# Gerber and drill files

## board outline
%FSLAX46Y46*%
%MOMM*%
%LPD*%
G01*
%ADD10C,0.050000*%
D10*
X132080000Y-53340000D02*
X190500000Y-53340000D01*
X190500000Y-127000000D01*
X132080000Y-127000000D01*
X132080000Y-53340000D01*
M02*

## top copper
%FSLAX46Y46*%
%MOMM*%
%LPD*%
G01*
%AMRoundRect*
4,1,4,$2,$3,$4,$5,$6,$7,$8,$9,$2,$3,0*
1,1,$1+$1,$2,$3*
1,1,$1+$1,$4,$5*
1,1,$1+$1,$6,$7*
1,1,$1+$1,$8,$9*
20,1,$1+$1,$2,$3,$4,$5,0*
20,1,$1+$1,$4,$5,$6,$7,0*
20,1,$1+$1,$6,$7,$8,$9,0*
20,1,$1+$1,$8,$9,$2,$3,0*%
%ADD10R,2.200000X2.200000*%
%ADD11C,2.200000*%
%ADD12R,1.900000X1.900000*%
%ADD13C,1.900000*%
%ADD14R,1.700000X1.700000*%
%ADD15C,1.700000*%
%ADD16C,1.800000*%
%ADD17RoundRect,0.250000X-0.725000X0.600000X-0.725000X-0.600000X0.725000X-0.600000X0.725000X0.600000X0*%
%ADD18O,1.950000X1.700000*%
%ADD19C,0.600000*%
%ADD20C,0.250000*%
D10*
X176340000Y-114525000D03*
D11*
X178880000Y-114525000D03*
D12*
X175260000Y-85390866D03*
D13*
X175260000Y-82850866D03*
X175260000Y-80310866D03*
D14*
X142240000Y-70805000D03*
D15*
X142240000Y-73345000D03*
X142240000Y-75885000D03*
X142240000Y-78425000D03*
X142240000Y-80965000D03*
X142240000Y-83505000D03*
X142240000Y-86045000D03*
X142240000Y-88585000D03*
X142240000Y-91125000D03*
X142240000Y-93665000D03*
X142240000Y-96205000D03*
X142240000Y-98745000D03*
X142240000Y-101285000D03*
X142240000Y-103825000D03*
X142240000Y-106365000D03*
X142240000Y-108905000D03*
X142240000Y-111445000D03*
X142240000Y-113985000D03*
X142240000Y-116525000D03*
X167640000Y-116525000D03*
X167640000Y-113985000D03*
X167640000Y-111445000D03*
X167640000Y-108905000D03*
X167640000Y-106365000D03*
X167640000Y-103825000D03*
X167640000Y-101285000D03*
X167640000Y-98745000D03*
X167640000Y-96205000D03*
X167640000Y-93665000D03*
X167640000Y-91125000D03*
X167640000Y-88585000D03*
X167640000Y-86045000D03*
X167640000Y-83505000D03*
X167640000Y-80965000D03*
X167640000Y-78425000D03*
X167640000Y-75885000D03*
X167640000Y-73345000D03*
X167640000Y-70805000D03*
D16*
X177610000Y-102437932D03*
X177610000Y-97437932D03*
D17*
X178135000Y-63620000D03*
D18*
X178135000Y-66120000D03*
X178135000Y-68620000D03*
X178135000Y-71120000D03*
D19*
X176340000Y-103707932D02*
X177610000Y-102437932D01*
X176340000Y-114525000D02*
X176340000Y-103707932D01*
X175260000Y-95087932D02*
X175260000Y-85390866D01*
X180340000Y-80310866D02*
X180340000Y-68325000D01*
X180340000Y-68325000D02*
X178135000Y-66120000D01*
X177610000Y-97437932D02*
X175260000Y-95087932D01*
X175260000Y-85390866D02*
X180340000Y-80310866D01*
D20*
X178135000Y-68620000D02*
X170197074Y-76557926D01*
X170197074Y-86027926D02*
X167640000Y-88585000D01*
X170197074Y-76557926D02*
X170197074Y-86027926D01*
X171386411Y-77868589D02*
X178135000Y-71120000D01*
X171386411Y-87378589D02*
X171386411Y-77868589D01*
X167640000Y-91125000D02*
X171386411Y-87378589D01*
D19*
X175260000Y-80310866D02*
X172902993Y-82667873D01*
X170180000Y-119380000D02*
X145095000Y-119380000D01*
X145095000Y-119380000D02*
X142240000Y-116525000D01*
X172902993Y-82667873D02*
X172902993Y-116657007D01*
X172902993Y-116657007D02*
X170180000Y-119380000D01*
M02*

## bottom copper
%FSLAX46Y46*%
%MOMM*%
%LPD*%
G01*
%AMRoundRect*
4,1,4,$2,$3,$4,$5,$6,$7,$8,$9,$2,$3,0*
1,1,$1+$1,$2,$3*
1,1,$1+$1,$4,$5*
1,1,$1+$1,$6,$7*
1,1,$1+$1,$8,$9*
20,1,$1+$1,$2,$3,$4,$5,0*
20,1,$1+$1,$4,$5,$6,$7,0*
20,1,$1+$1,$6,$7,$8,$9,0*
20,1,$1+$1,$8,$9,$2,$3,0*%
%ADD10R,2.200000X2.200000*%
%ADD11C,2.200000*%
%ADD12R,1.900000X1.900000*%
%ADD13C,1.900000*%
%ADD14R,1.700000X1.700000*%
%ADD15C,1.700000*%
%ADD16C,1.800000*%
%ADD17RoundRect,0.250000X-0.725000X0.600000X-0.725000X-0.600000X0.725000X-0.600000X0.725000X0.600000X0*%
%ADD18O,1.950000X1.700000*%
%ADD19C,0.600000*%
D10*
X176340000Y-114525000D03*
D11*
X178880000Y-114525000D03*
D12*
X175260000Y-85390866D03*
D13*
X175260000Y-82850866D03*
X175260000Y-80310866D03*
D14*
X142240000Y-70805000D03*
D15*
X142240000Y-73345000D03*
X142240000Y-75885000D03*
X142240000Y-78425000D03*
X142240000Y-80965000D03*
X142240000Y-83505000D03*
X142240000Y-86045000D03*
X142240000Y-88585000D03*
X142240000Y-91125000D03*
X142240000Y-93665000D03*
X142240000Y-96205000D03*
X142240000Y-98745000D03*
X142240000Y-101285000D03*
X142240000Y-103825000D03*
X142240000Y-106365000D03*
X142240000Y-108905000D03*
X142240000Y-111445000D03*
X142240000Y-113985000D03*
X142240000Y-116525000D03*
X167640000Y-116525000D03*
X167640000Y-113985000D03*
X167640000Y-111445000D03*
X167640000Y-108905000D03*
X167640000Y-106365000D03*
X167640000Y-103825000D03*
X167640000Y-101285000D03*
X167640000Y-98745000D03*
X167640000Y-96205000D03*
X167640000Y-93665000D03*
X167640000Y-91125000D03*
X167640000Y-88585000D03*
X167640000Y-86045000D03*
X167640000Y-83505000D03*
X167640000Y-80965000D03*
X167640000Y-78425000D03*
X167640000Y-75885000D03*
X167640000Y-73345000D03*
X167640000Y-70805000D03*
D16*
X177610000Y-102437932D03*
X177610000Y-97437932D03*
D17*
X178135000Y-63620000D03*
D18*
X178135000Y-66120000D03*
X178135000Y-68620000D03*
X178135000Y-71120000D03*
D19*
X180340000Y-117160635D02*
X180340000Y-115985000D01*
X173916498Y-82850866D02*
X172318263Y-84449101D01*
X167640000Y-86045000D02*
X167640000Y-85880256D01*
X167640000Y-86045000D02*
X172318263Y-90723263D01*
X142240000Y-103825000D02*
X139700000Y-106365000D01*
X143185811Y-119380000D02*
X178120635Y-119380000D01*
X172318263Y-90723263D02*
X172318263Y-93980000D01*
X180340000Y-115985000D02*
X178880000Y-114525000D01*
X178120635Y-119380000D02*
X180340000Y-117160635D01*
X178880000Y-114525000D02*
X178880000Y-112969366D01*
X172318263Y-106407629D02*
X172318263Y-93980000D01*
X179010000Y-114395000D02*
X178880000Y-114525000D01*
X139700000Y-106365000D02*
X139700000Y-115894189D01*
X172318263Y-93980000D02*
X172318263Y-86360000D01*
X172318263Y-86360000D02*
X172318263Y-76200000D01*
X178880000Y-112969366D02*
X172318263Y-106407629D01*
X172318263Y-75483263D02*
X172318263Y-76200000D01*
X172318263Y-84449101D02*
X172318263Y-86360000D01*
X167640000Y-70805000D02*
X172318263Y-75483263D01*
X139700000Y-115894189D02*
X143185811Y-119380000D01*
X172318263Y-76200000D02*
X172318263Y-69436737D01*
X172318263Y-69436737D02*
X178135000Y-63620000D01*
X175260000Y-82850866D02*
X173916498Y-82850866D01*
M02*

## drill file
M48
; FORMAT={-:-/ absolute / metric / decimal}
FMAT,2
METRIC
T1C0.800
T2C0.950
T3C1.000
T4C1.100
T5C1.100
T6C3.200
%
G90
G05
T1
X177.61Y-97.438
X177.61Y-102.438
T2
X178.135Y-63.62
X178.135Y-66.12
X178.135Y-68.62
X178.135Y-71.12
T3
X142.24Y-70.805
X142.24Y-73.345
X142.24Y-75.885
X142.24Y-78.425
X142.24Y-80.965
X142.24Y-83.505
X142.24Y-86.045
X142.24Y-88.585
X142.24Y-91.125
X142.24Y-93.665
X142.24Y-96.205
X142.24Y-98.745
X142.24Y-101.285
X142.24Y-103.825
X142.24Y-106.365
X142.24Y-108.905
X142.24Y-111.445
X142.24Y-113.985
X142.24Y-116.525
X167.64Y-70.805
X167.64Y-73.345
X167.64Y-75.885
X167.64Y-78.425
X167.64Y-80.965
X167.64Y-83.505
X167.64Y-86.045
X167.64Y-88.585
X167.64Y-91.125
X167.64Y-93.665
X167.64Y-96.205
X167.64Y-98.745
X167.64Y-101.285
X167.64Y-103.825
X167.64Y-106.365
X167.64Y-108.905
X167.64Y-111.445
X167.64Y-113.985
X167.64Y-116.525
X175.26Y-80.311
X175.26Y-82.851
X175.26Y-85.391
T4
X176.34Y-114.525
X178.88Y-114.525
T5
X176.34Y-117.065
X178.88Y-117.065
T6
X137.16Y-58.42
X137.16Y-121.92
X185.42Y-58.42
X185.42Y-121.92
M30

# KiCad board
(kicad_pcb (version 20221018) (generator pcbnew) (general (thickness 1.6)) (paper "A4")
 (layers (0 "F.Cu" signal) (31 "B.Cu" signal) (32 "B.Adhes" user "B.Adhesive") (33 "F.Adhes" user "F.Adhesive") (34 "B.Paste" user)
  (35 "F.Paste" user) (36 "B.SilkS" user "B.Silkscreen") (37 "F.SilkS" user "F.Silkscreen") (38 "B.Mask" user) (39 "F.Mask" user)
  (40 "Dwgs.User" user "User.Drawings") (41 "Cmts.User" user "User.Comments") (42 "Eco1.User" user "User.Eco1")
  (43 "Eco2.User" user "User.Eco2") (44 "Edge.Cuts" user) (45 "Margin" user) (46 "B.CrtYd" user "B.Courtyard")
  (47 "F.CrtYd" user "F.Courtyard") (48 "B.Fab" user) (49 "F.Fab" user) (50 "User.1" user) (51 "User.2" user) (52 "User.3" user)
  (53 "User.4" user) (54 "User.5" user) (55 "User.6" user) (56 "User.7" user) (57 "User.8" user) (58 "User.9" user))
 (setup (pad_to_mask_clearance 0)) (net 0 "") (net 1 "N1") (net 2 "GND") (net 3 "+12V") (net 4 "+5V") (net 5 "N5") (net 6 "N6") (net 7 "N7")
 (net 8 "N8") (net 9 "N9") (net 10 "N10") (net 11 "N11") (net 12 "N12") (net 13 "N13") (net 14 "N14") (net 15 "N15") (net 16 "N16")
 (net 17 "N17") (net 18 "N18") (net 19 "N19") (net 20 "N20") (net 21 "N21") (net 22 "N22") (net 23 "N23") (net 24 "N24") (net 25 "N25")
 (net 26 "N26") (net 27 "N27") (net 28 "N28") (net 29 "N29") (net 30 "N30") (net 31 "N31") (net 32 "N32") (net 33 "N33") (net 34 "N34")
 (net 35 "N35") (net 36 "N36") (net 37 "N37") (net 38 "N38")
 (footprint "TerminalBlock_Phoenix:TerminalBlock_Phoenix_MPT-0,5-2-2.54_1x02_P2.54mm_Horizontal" (layer "F.Cu") (at 176.34 114.525)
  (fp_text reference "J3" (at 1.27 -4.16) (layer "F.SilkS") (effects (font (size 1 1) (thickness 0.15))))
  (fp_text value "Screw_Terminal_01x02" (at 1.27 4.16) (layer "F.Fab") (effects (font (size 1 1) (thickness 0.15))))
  (pad "" np_thru_hole circle (at 0 2.54) (size 1.1 1.1) (drill 1.1) (layers "*.Cu" "*.Mask"))
  (pad "" np_thru_hole circle (at 2.54 2.54) (size 1.1 1.1) (drill 1.1) (layers "*.Cu" "*.Mask"))
  (pad "1" thru_hole rect (at 0 0) (size 2.2 2.2) (drill 1.1) (layers "*.Cu" "*.Mask") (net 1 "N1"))
  (pad "2" thru_hole circle (at 2.54 0) (size 2.2 2.2) (drill 1.1) (layers "*.Cu" "*.Mask") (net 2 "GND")))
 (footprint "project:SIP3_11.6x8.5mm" (layer "F.Cu") (at 175.26 85.390866 90)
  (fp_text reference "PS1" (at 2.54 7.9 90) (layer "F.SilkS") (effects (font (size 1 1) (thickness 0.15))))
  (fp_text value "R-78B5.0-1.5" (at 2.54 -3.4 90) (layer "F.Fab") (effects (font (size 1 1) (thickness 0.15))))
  (pad "1" thru_hole rect (at 0 0) (size 1.9 1.9) (drill 1) (layers "*.Cu" "*.Mask") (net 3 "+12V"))
  (pad "2" thru_hole circle (at 2.54 0 270) (size 1.9 1.9) (drill 1) (layers "*.Cu" "*.Mask") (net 2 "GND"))
  (pad "3" thru_hole circle (at 5.08 0) (size 1.9 1.9) (drill 1) (layers "*.Cu" "*.Mask") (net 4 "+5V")))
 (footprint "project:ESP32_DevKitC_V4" (layer "F.Cu") (at 142.24 70.805)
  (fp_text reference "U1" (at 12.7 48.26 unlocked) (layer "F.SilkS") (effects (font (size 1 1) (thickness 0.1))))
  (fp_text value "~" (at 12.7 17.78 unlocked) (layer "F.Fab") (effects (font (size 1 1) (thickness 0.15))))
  (pad "1" thru_hole rect (at 0 0 270) (size 1.7 1.7) (drill 1) (layers "*.Cu" "*.Mask") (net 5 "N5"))
  (pad "2" thru_hole circle (at 0 2.54 270) (size 1.7 1.7) (drill 1) (layers "*.Cu" "*.Mask") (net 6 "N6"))
  (pad "3" thru_hole circle (at 0 5.08 270) (size 1.7 1.7) (drill 1) (layers "*.Cu" "*.Mask") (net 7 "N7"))
  (pad "4" thru_hole circle (at 0 7.62 270) (size 1.7 1.7) (drill 1) (layers "*.Cu" "*.Mask") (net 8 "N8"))
  (pad "5" thru_hole circle (at 0 10.16 270) (size 1.7 1.7) (drill 1) (layers "*.Cu" "*.Mask") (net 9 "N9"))
  (pad "6" thru_hole circle (at 0 12.7 270) (size 1.7 1.7) (drill 1) (layers "*.Cu" "*.Mask") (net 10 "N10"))
  (pad "7" thru_hole circle (at 0 15.24 270) (size 1.7 1.7) (drill 1) (layers "*.Cu" "*.Mask") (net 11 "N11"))
  (pad "8" thru_hole circle (at 0 17.78 270) (size 1.7 1.7) (drill 1) (layers "*.Cu" "*.Mask") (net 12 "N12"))
  (pad "9" thru_hole circle (at 0 20.32 270) (size 1.7 1.7) (drill 1) (layers "*.Cu" "*.Mask") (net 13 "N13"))
  (pad "10" thru_hole circle (at 0 22.86 270) (size 1.7 1.7) (drill 1) (layers "*.Cu" "*.Mask") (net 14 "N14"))
  (pad "11" thru_hole circle (at 0 25.4 270) (size 1.7 1.7) (drill 1) (layers "*.Cu" "*.Mask") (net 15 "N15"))
  (pad "12" thru_hole circle (at 0 27.94 270) (size 1.7 1.7) (drill 1) (layers "*.Cu" "*.Mask") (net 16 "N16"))
  (pad "13" thru_hole circle (at 0 30.48 270) (size 1.7 1.7) (drill 1) (layers "*.Cu" "*.Mask") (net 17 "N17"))
  (pad "14" thru_hole circle (at 0 33.02 270) (size 1.7 1.7) (drill 1) (layers "*.Cu" "*.Mask") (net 2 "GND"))
  (pad "15" thru_hole circle (at 0 35.56 270) (size 1.7 1.7) (drill 1) (layers "*.Cu" "*.Mask") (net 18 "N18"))
  (pad "16" thru_hole circle (at 0 38.1 270) (size 1.7 1.7) (drill 1) (layers "*.Cu" "*.Mask") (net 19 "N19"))
  (pad "17" thru_hole circle (at 0 40.64 270) (size 1.7 1.7) (drill 1) (layers "*.Cu" "*.Mask") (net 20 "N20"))
  (pad "18" thru_hole circle (at 0 43.18 270) (size 1.7 1.7) (drill 1) (layers "*.Cu" "*.Mask") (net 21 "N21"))
  (pad "19" thru_hole circle (at 0 45.72 270) (size 1.7 1.7) (drill 1) (layers "*.Cu" "*.Mask") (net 4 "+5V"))
  (pad "20" thru_hole circle (at 25.4 45.72 270) (size 1.7 1.7) (drill 1) (layers "*.Cu" "*.Mask") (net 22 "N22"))
  (pad "21" thru_hole circle (at 25.4 43.18 270) (size 1.7 1.7) (drill 1) (layers "*.Cu" "*.Mask") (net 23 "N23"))
  (pad "22" thru_hole circle (at 25.4 40.64 270) (size 1.7 1.7) (drill 1) (layers "*.Cu" "*.Mask") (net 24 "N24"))
  (pad "23" thru_hole circle (at 25.4 38.1 270) (size 1.7 1.7) (drill 1) (layers "*.Cu" "*.Mask") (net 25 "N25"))
  (pad "24" thru_hole circle (at 25.4 35.56 270) (size 1.7 1.7) (drill 1) (layers "*.Cu" "*.Mask") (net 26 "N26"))
  (pad "25" thru_hole circle (at 25.4 33.02 270) (size 1.7 1.7) (drill 1) (layers "*.Cu" "*.Mask") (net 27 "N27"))
  (pad "26" thru_hole circle (at 25.4 30.48 270) (size 1.7 1.7) (drill 1) (layers "*.Cu" "*.Mask") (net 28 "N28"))
  (pad "27" thru_hole circle (at 25.4 27.94 270) (size 1.7 1.7) (drill 1) (layers "*.Cu" "*.Mask") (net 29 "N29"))
  (pad "28" thru_hole circle (at 25.4 25.4 270) (size 1.7 1.7) (drill 1) (layers "*.Cu" "*.Mask") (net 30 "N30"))
  (pad "29" thru_hole circle (at 25.4 22.86 270) (size 1.7 1.7) (drill 1) (layers "*.Cu" "*.Mask") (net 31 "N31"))
  (pad "30" thru_hole circle (at 25.4 20.32 270) (size 1.7 1.7) (drill 1) (layers "*.Cu" "*.Mask") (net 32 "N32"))
  (pad "31" thru_hole circle (at 25.4 17.78 270) (size 1.7 1.7) (drill 1) (layers "*.Cu" "*.Mask") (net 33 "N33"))
  (pad "32" thru_hole circle (at 25.4 15.24 270) (size 1.7 1.7) (drill 1) (layers "*.Cu" "*.Mask") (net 2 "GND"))
  (pad "33" thru_hole circle (at 25.4 12.7 270) (size 1.7 1.7) (drill 1) (layers "*.Cu" "*.Mask") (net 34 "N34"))
  (pad "34" thru_hole circle (at 25.4 10.16 270) (size 1.7 1.7) (drill 1) (layers "*.Cu" "*.Mask") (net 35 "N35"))
  (pad "35" thru_hole circle (at 25.4 7.62 270) (size 1.7 1.7) (drill 1) (layers "*.Cu" "*.Mask") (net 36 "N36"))
  (pad "36" thru_hole circle (at 25.4 5.08 270) (size 1.7 1.7) (drill 1) (layers "*.Cu" "*.Mask") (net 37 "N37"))
  (pad "37" thru_hole circle (at 25.4 2.54 270) (size 1.7 1.7) (drill 1) (layers "*.Cu" "*.Mask") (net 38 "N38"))
  (pad "38" thru_hole circle (at 25.4 0 270) (size 1.7 1.7) (drill 1) (layers "*.Cu" "*.Mask") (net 2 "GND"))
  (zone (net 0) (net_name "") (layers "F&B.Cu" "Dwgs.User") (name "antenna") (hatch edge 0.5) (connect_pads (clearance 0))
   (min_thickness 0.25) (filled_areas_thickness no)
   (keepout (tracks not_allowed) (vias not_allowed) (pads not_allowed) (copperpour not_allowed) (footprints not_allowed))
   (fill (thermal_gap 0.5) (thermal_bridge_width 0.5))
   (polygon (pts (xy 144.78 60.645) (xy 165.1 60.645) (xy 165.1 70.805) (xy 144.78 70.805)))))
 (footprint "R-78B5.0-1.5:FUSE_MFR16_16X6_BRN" (layer "F.Cu") (at 177.61 102.437932 90)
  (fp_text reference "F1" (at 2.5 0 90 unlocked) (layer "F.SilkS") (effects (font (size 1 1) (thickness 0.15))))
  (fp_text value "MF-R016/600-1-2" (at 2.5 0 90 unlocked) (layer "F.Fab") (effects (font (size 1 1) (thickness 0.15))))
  (pad "1" thru_hole circle (at 0 0 90) (size 1.8 1.8) (drill 0.8) (layers "*.Cu" "*.Mask") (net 1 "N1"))
  (pad "2" thru_hole circle (at 5 0 90) (size 1.8 1.8) (drill 0.8) (layers "*.Cu" "*.Mask") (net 3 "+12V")))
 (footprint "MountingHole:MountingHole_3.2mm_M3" (layer "F.Cu") (at 185.42 58.42)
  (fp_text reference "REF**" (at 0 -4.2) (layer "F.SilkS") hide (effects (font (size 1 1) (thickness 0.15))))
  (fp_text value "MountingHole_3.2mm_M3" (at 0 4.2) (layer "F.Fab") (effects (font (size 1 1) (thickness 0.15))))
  (pad "" np_thru_hole circle (at 0 0) (size 3.2 3.2) (drill 3.2) (layers "*.Cu" "*.Mask")))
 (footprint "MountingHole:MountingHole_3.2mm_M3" (layer "F.Cu") (at 137.16 121.92)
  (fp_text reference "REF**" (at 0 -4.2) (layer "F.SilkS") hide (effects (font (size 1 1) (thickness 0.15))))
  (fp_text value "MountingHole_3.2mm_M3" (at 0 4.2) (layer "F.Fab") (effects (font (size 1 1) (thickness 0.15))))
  (pad "" np_thru_hole circle (at 0 0) (size 3.2 3.2) (drill 3.2) (layers "F&B.Cu" "*.Mask")))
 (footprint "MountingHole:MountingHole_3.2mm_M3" (layer "F.Cu") (at 137.16 58.42)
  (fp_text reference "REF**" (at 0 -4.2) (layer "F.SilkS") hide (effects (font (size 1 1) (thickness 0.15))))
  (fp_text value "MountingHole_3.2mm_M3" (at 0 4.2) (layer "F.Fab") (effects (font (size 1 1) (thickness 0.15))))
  (pad "" np_thru_hole circle (at 0 0) (size 3.2 3.2) (drill 3.2) (layers "F&B.Cu" "*.Mask")))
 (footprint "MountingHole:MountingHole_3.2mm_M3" (layer "F.Cu") (at 185.42 121.92)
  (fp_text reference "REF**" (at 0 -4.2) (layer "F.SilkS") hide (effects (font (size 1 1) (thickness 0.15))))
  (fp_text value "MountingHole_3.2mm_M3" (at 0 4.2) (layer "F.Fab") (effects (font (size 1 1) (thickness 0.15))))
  (pad "" np_thru_hole circle (at 0 0) (size 3.2 3.2) (drill 3.2) (layers "F&B.Cu" "*.Mask")))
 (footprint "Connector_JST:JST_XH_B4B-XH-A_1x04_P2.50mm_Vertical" (layer "F.Cu") (at 178.135 63.62 -90)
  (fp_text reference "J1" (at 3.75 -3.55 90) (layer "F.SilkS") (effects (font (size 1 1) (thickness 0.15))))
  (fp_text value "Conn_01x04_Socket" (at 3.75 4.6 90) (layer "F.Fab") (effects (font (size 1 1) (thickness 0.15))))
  (pad "1" thru_hole roundrect (at 0 0 270) (size 1.7 1.95) (drill 0.95) (layers "*.Cu" "*.Mask") (roundrect_rratio 0.1470588235)
   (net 2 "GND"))
  (pad "2" thru_hole oval (at 2.5 0 270) (size 1.7 1.95) (drill 0.95) (layers "*.Cu" "*.Mask") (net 3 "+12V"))
  (pad "3" thru_hole oval (at 5 0 270) (size 1.7 1.95) (drill 0.95) (layers "*.Cu" "*.Mask") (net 33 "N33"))
  (pad "4" thru_hole oval (at 7.5 0 270) (size 1.7 1.95) (drill 0.95) (layers "*.Cu" "*.Mask") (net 32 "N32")))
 (gr_rect (start 132.08 53.34) (end 190.5 127) (stroke (width 0.05) (type default)) (fill none) (layer "Edge.Cuts"))
 (segment (start 176.34 103.707932) (end 177.61 102.437932) (width 0.6) (layer "F.Cu") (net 1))
 (segment (start 176.34 114.525) (end 176.34 103.707932) (width 0.6) (layer "F.Cu") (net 1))
 (segment (start 175.26 95.087932) (end 175.26 85.390866) (width 0.6) (layer "F.Cu") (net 3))
 (segment (start 180.34 80.310866) (end 180.34 68.325) (width 0.6) (layer "F.Cu") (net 3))
 (segment (start 180.34 68.325) (end 178.135 66.12) (width 0.6) (layer "F.Cu") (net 3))
 (segment (start 177.61 97.437932) (end 175.26 95.087932) (width 0.6) (layer "F.Cu") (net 3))
 (segment (start 175.26 85.390866) (end 180.34 80.310866) (width 0.6) (layer "F.Cu") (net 3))
 (segment (start 180.34 117.160635) (end 180.34 115.985) (width 0.6) (layer "B.Cu") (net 2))
 (segment (start 173.916498 82.850866) (end 172.318263 84.449101) (width 0.6) (layer "B.Cu") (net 2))
 (segment (start 167.64 86.045) (end 167.64 85.880256) (width 0.6) (layer "B.Cu") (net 2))
 (segment (start 167.64 86.045) (end 172.318263 90.723263) (width 0.6) (layer "B.Cu") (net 2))
 (segment (start 142.24 103.825) (end 139.7 106.365) (width 0.6) (layer "B.Cu") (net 2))
 (segment (start 143.185811 119.38) (end 178.120635 119.38) (width 0.6) (layer "B.Cu") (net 2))
 (segment (start 172.318263 90.723263) (end 172.318263 93.98) (width 0.6) (layer "B.Cu") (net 2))
 (segment (start 180.34 115.985) (end 178.88 114.525) (width 0.6) (layer "B.Cu") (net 2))
 (segment (start 178.120635 119.38) (end 180.34 117.160635) (width 0.6) (layer "B.Cu") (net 2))
 (segment (start 178.88 114.525) (end 178.88 112.969366) (width 0.6) (layer "B.Cu") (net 2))
 (segment (start 172.318263 106.407629) (end 172.318263 93.98) (width 0.6) (layer "B.Cu") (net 2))
 (segment (start 179.01 114.395) (end 178.88 114.525) (width 0.6) (layer "B.Cu") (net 2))
 (segment (start 139.7 106.365) (end 139.7 115.894189) (width 0.6) (layer "B.Cu") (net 2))
 (segment (start 172.318263 93.98) (end 172.318263 86.36) (width 0.6) (layer "B.Cu") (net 2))
 (segment (start 172.318263 86.36) (end 172.318263 76.2) (width 0.6) (layer "B.Cu") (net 2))
 (segment (start 178.88 112.969366) (end 172.318263 106.407629) (width 0.6) (layer "B.Cu") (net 2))
 (segment (start 172.318263 75.483263) (end 172.318263 76.2) (width 0.6) (layer "B.Cu") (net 2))
 (segment (start 172.318263 84.449101) (end 172.318263 86.36) (width 0.6) (layer "B.Cu") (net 2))
 (segment (start 167.64 70.805) (end 172.318263 75.483263) (width 0.6) (layer "B.Cu") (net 2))
 (segment (start 139.7 115.894189) (end 143.185811 119.38) (width 0.6) (layer "B.Cu") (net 2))
 (segment (start 172.318263 76.2) (end 172.318263 69.436737) (width 0.6) (layer "B.Cu") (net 2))
 (segment (start 172.318263 69.436737) (end 178.135 63.62) (width 0.6) (layer "B.Cu") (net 2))
 (segment (start 175.26 82.850866) (end 173.916498 82.850866) (width 0.6) (layer "B.Cu") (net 2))
 (segment (start 178.135 68.62) (end 170.197074 76.557926) (width 0.25) (layer "F.Cu") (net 33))
 (segment (start 170.197074 86.027926) (end 167.64 88.585) (width 0.25) (layer "F.Cu") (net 33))
 (segment (start 170.197074 76.557926) (end 170.197074 86.027926) (width 0.25) (layer "F.Cu") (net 33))
 (segment (start 171.386411 77.868589) (end 178.135 71.12) (width 0.25) (layer "F.Cu") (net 32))
 (segment (start 171.386411 87.378589) (end 171.386411 77.868589) (width 0.25) (layer "F.Cu") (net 32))
 (segment (start 167.64 91.125) (end 171.386411 87.378589) (width 0.25) (layer "F.Cu") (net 32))
 (segment (start 175.26 80.310866) (end 172.902993 82.667873) (width 0.6) (layer "F.Cu") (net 4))
 (segment (start 170.18 119.38) (end 145.095 119.38) (width 0.6) (layer "F.Cu") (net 4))
 (segment (start 145.095 119.38) (end 142.24 116.525) (width 0.6) (layer "F.Cu") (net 4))
 (segment (start 172.902993 82.667873) (end 172.902993 116.657007) (width 0.6) (layer "F.Cu") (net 4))
 (segment (start 172.902993 116.657007) (end 170.18 119.38) (width 0.6) (layer "F.Cu") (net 4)))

